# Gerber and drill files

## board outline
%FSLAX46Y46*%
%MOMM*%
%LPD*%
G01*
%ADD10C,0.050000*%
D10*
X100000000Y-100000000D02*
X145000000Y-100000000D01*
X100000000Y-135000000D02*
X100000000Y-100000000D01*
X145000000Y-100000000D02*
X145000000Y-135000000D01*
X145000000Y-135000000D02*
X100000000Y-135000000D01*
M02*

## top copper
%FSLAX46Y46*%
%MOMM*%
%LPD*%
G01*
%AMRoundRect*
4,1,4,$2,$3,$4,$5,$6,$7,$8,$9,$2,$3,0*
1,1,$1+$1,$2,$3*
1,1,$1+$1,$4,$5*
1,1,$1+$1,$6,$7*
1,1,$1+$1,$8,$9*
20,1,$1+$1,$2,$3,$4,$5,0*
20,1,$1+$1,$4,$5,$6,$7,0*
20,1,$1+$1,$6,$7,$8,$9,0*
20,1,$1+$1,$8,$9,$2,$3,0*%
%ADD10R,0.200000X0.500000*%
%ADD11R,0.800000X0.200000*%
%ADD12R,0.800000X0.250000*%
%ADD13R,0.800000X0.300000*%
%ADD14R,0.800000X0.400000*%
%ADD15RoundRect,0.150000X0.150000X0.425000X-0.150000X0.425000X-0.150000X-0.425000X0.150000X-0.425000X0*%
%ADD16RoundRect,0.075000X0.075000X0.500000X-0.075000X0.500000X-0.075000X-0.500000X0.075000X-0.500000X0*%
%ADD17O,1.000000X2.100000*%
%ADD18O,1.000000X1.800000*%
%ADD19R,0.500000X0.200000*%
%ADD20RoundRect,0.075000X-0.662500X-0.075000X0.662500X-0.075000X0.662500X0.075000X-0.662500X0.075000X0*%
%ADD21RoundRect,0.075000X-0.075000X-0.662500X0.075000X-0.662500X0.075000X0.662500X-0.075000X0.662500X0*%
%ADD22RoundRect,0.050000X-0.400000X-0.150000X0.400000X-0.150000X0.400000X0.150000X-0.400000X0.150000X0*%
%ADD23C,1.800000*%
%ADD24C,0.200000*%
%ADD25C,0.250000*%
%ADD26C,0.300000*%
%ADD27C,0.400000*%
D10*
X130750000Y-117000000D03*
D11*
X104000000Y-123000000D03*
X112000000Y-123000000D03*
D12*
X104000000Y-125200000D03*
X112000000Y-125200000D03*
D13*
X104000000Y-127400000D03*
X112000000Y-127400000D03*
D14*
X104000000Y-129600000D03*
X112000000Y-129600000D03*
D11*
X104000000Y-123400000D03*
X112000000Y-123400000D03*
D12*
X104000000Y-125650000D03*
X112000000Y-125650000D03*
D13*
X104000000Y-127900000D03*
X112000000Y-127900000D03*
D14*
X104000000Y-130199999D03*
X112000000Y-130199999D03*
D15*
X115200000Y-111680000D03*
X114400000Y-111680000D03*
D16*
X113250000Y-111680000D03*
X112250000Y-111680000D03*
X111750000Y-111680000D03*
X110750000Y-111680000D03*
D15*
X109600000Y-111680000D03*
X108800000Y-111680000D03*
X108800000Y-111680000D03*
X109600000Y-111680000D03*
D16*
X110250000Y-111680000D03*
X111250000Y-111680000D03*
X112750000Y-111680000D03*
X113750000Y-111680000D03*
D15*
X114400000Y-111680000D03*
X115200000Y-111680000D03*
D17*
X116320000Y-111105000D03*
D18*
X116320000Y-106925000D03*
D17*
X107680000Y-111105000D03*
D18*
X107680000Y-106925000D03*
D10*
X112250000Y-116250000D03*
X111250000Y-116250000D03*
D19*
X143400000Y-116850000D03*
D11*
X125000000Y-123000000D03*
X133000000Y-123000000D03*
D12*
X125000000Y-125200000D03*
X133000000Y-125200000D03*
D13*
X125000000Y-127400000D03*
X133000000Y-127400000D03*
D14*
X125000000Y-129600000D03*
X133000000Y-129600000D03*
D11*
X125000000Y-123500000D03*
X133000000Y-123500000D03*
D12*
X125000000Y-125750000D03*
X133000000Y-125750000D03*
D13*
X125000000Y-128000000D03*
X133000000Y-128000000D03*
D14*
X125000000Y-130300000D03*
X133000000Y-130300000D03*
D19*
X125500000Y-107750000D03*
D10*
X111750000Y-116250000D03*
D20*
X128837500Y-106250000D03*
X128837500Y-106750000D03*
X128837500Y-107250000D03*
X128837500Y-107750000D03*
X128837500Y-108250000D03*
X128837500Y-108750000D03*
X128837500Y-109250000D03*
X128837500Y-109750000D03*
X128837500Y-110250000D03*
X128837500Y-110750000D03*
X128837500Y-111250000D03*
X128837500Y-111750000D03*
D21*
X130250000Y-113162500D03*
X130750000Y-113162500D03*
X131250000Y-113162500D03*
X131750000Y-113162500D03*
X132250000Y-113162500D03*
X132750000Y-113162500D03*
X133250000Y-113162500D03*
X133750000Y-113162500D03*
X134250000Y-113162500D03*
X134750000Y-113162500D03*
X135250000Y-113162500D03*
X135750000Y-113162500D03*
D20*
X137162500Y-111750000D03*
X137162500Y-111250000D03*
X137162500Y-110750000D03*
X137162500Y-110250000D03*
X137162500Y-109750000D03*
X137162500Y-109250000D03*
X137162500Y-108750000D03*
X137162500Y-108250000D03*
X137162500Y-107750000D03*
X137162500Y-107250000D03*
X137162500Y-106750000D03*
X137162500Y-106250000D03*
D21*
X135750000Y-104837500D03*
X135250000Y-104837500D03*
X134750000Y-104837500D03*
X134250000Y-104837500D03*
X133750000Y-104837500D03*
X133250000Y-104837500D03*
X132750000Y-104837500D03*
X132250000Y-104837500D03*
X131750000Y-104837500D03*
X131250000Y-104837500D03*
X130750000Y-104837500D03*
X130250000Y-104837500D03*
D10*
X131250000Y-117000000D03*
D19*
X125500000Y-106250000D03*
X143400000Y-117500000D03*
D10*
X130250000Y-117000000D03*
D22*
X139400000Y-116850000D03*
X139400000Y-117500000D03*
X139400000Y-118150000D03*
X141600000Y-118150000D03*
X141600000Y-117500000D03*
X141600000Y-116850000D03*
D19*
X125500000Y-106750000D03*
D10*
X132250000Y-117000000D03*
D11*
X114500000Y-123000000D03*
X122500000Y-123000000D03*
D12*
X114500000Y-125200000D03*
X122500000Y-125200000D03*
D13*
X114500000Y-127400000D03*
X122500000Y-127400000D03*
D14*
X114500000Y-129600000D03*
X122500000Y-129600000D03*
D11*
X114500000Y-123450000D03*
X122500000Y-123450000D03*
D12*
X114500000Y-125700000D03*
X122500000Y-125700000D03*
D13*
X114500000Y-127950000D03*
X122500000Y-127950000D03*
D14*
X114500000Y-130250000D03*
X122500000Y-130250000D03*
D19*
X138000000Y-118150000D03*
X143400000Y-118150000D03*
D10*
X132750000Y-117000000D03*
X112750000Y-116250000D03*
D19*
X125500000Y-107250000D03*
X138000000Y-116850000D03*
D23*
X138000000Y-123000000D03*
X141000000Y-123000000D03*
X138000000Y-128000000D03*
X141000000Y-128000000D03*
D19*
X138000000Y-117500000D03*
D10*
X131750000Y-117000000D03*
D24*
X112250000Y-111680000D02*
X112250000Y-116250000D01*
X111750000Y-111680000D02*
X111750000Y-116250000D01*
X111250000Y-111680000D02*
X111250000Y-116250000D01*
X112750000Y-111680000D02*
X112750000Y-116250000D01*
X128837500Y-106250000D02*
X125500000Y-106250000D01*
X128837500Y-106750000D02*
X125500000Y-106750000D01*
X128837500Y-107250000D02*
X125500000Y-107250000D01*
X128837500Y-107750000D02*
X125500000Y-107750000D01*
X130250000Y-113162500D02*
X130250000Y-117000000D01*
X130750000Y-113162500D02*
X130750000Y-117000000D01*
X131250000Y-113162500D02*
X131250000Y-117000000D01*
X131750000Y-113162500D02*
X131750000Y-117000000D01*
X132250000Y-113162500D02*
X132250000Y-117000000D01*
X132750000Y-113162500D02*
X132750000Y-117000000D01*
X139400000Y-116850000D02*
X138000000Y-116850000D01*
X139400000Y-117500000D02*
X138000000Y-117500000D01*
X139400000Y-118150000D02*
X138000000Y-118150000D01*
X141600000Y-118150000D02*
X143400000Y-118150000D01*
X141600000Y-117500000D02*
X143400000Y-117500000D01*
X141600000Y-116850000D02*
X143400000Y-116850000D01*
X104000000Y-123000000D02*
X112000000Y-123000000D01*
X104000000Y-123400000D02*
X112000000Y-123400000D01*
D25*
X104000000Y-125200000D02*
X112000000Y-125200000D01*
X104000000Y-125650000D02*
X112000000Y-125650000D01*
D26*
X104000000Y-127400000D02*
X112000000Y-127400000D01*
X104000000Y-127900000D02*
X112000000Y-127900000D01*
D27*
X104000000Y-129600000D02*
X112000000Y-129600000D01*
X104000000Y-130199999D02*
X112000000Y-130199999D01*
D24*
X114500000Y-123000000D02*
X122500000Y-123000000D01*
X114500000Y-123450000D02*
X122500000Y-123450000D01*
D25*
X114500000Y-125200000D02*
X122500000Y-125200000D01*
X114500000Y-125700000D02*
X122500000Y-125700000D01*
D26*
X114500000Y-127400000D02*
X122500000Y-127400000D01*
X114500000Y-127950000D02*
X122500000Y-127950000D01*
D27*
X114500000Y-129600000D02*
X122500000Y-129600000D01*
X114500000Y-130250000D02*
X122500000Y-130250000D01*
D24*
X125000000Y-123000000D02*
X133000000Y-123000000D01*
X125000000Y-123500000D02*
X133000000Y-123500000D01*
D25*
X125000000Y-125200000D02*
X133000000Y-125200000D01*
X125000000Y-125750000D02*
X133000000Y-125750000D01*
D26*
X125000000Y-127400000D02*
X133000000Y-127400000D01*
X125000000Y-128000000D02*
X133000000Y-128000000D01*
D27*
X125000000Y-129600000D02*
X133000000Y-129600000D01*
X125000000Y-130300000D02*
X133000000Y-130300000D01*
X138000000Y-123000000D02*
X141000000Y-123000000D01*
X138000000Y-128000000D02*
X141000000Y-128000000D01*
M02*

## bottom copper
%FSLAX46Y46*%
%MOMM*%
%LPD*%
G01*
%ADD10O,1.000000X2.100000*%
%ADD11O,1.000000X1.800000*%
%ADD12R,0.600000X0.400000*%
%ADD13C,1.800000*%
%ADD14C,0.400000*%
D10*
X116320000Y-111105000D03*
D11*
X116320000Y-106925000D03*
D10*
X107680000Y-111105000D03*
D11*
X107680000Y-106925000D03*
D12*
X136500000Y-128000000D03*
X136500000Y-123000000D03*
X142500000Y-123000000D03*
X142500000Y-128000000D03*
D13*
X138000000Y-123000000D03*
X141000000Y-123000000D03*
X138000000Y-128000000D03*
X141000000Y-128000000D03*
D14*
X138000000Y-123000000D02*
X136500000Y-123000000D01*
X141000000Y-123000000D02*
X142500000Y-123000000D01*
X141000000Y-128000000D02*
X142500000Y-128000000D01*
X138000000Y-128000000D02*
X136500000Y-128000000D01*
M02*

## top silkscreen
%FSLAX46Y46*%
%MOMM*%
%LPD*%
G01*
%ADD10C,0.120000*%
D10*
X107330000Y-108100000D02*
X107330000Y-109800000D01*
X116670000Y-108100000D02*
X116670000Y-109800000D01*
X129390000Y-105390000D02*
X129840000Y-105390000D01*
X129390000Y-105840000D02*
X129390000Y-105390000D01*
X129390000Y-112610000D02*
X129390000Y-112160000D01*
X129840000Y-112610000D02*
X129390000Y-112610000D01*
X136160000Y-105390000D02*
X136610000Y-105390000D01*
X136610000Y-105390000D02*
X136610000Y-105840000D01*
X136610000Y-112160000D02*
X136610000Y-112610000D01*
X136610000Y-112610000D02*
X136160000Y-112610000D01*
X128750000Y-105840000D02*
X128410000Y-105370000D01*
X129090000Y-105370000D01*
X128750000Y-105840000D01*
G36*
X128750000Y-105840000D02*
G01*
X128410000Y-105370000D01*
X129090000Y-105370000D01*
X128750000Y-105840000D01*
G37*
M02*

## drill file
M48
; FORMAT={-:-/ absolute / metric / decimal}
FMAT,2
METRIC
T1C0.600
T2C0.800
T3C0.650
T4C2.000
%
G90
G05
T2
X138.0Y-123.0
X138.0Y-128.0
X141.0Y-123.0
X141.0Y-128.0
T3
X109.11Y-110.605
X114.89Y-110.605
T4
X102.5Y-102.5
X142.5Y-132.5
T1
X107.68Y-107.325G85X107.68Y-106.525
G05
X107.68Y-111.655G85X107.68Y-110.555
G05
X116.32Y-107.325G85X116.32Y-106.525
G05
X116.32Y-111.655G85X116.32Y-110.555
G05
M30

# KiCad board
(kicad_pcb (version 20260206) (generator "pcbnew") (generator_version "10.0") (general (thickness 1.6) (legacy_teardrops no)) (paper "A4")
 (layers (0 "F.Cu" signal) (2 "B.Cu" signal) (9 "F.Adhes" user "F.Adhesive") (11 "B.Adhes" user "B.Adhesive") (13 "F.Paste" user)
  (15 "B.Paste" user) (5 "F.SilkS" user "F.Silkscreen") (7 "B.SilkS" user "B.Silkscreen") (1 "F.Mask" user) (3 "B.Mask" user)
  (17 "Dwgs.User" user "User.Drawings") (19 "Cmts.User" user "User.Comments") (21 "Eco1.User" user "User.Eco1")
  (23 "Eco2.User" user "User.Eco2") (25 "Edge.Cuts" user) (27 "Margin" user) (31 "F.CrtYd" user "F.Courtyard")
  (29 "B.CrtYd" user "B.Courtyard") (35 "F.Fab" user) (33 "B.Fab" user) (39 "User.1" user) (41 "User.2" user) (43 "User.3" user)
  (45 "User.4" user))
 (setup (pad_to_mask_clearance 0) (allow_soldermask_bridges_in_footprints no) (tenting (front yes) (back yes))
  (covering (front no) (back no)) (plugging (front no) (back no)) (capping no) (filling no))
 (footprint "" (layer "F.Cu") (at 0 0)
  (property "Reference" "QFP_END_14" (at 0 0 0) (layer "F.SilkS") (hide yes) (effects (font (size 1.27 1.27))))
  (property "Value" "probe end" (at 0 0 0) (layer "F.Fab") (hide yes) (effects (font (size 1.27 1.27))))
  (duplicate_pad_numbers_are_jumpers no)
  (pad "1" smd rect (at 130.75 117) (size 0.2 0.5) (layers "F.Cu" "F.Mask") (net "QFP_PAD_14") (thermal_bridge_angle 45)))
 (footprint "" (layer "F.Cu") (at 0 0)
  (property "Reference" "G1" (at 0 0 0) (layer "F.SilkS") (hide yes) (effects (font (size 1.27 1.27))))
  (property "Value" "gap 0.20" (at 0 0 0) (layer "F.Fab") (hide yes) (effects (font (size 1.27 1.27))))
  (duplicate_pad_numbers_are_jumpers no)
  (pad "A0L" smd rect (at 104 123) (size 0.8 0.2) (layers "F.Cu" "F.Mask" "F.Paste") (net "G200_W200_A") (thermal_bridge_angle 45))
  (pad "A0R" smd rect (at 112 123) (size 0.8 0.2) (layers "F.Cu" "F.Mask" "F.Paste") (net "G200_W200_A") (thermal_bridge_angle 45))
  (pad "A1L" smd rect (at 104 125.2) (size 0.8 0.25) (layers "F.Cu" "F.Mask" "F.Paste") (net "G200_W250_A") (thermal_bridge_angle 45))
  (pad "A1R" smd rect (at 112 125.2) (size 0.8 0.25) (layers "F.Cu" "F.Mask" "F.Paste") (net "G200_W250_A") (thermal_bridge_angle 45))
  (pad "A2L" smd rect (at 104 127.4) (size 0.8 0.3) (layers "F.Cu" "F.Mask" "F.Paste") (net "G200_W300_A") (thermal_bridge_angle 45))
  (pad "A2R" smd rect (at 112 127.4) (size 0.8 0.3) (layers "F.Cu" "F.Mask" "F.Paste") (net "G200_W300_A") (thermal_bridge_angle 45))
  (pad "A3L" smd rect (at 104 129.6) (size 0.8 0.4) (layers "F.Cu" "F.Mask" "F.Paste") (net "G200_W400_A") (thermal_bridge_angle 45))
  (pad "A3R" smd rect (at 112 129.6) (size 0.8 0.4) (layers "F.Cu" "F.Mask" "F.Paste") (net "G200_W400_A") (thermal_bridge_angle 45))
  (pad "B0L" smd rect (at 104 123.4) (size 0.8 0.2) (layers "F.Cu" "F.Mask" "F.Paste") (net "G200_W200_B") (thermal_bridge_angle 45))
  (pad "B0R" smd rect (at 112 123.4) (size 0.8 0.2) (layers "F.Cu" "F.Mask" "F.Paste") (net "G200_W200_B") (thermal_bridge_angle 45))
  (pad "B1L" smd rect (at 104 125.65) (size 0.8 0.25) (layers "F.Cu" "F.Mask" "F.Paste") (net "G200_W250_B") (thermal_bridge_angle 45))
  (pad "B1R" smd rect (at 112 125.65) (size 0.8 0.25) (layers "F.Cu" "F.Mask" "F.Paste") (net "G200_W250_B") (thermal_bridge_angle 45))
  (pad "B2L" smd rect (at 104 127.9) (size 0.8 0.3) (layers "F.Cu" "F.Mask" "F.Paste") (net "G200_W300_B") (thermal_bridge_angle 45))
  (pad "B2R" smd rect (at 112 127.9) (size 0.8 0.3) (layers "F.Cu" "F.Mask" "F.Paste") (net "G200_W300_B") (thermal_bridge_angle 45))
  (pad "B3L" smd rect (at 104 130.199999) (size 0.8 0.4) (layers "F.Cu" "F.Mask" "F.Paste") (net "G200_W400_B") (thermal_bridge_angle 45))
  (pad "B3R" smd rect (at 112 130.199999) (size 0.8 0.4) (layers "F.Cu" "F.Mask" "F.Paste") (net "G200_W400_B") (thermal_bridge_angle 45)))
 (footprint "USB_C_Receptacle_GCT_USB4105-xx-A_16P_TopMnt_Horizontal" (layer "F.Cu") (at 112 108 180)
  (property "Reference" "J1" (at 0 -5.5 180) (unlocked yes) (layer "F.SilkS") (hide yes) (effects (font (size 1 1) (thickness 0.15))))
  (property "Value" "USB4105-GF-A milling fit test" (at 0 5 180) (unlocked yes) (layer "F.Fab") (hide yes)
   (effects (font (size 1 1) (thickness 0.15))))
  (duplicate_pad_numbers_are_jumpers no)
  (fp_line (start 4.67 -0.1) (end 4.67 -1.8) (stroke (width 0.12) (type solid)) (layer "F.SilkS"))
  (fp_line (start -4.67 -0.1) (end -4.67 -1.8) (stroke (width 0.12) (type solid)) (layer "F.SilkS"))
  (pad "" np_thru_hole circle (at -2.89 -2.605 180) (size 0.65 0.65) (drill 0.65) (layers "*.Cu" "*.Mask"))
  (pad "" np_thru_hole circle (at 2.89 -2.605 180) (size 0.65 0.65) (drill 0.65) (layers "*.Cu" "*.Mask"))
  (pad "A1" smd roundrect (at -3.2 -3.68 180) (size 0.6 1.15) (layers "F.Cu" "F.Mask" "F.Paste") (roundrect_rratio 0.25)
   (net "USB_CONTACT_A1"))
  (pad "A4" smd roundrect (at -2.4 -3.68 180) (size 0.6 1.15) (layers "F.Cu" "F.Mask" "F.Paste") (roundrect_rratio 0.25)
   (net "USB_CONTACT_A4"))
  (pad "A5" smd roundrect (at -1.25 -3.68 180) (size 0.3 1.15) (layers "F.Cu" "F.Mask" "F.Paste") (roundrect_rratio 0.25)
   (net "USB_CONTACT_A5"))
  (pad "A6" smd roundrect (at -0.25 -3.68 180) (size 0.3 1.15) (layers "F.Cu" "F.Mask" "F.Paste") (roundrect_rratio 0.25)
   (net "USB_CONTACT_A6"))
  (pad "A7" smd roundrect (at 0.25 -3.68 180) (size 0.3 1.15) (layers "F.Cu" "F.Mask" "F.Paste") (roundrect_rratio 0.25)
   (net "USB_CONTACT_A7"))
  (pad "A8" smd roundrect (at 1.25 -3.68 180) (size 0.3 1.15) (layers "F.Cu" "F.Mask" "F.Paste") (roundrect_rratio 0.25)
   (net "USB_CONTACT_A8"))
  (pad "A9" smd roundrect (at 2.4 -3.68 180) (size 0.6 1.15) (layers "F.Cu" "F.Mask" "F.Paste") (roundrect_rratio 0.25)
   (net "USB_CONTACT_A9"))
  (pad "A12" smd roundrect (at 3.2 -3.68 180) (size 0.6 1.15) (layers "F.Cu" "F.Mask" "F.Paste") (roundrect_rratio 0.25)
   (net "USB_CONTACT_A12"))
  (pad "B1" smd roundrect (at 3.2 -3.68 180) (size 0.6 1.15) (layers "F.Cu" "F.Mask" "F.Paste") (roundrect_rratio 0.25)
   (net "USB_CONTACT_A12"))
  (pad "B4" smd roundrect (at 2.4 -3.68 180) (size 0.6 1.15) (layers "F.Cu" "F.Mask" "F.Paste") (roundrect_rratio 0.25)
   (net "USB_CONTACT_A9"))
  (pad "B5" smd roundrect (at 1.75 -3.68 180) (size 0.3 1.15) (layers "F.Cu" "F.Mask" "F.Paste") (roundrect_rratio 0.25)
   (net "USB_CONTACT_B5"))
  (pad "B6" smd roundrect (at 0.75 -3.68 180) (size 0.3 1.15) (layers "F.Cu" "F.Mask" "F.Paste") (roundrect_rratio 0.25)
   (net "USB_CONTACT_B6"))
  (pad "B7" smd roundrect (at -0.75 -3.68 180) (size 0.3 1.15) (layers "F.Cu" "F.Mask" "F.Paste") (roundrect_rratio 0.25)
   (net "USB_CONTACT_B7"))
  (pad "B8" smd roundrect (at -1.75 -3.68 180) (size 0.3 1.15) (layers "F.Cu" "F.Mask" "F.Paste") (roundrect_rratio 0.25)
   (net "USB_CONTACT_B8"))
  (pad "B9" smd roundrect (at -2.4 -3.68 180) (size 0.6 1.15) (layers "F.Cu" "F.Mask" "F.Paste") (roundrect_rratio 0.25)
   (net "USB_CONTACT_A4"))
  (pad "B12" smd roundrect (at -3.2 -3.68 180) (size 0.6 1.15) (layers "F.Cu" "F.Mask" "F.Paste") (roundrect_rratio 0.25)
   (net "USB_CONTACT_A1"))
  (pad "SH" thru_hole oval (at -4.32 -3.105 180) (size 1 2.1) (drill oval 0.6 1.7) (layers "*.Cu" "*.Mask" "F.Paste")
   (remove_unused_layers no))
  (pad "SH" thru_hole oval (at -4.32 1.075 180) (size 1 1.8) (drill oval 0.6 1.4) (layers "*.Cu" "*.Mask" "F.Paste")
   (remove_unused_layers no))
  (pad "SH" thru_hole oval (at 4.32 -3.105 180) (size 1 2.1) (drill oval 0.6 1.7) (layers "*.Cu" "*.Mask" "F.Paste")
   (remove_unused_layers no))
  (pad "SH" thru_hole oval (at 4.32 1.075 180) (size 1 1.8) (drill oval 0.6 1.4) (layers "*.Cu" "*.Mask" "F.Paste")
   (remove_unused_layers no)))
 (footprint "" (layer "F.Cu") (at 0 0)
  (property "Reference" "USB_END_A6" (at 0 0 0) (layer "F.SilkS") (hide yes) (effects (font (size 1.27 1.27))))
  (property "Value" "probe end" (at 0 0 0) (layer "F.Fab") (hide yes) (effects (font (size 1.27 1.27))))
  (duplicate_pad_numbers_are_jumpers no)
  (pad "1" smd rect (at 112.25 116.25) (size 0.2 0.5) (layers "F.Cu" "F.Mask") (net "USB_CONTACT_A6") (thermal_bridge_angle 45)))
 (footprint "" (layer "F.Cu") (at 0 0)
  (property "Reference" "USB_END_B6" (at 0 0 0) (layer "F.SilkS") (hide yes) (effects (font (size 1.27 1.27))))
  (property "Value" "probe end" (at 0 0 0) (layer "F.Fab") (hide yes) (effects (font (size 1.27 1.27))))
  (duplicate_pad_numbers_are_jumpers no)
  (pad "1" smd rect (at 111.25 116.25) (size 0.2 0.5) (layers "F.Cu" "F.Mask") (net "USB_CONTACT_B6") (thermal_bridge_angle 45)))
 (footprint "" (layer "F.Cu") (at 0 0)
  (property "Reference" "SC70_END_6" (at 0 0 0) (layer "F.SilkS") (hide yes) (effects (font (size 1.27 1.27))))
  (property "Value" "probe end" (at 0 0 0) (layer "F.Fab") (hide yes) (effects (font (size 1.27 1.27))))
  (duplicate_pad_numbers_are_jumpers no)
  (pad "1" smd rect (at 143.4 116.85) (size 0.5 0.2) (layers "F.Cu" "F.Mask") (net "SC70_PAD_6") (thermal_bridge_angle 45)))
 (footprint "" (layer "F.Cu") (at 0 0)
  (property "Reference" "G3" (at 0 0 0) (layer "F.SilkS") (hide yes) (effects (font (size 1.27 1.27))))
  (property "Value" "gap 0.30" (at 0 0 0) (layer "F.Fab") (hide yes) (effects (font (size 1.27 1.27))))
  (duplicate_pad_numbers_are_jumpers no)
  (pad "A0L" smd rect (at 125 123) (size 0.8 0.2) (layers "F.Cu" "F.Mask" "F.Paste") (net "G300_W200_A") (thermal_bridge_angle 45))
  (pad "A0R" smd rect (at 133 123) (size 0.8 0.2) (layers "F.Cu" "F.Mask" "F.Paste") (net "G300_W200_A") (thermal_bridge_angle 45))
  (pad "A1L" smd rect (at 125 125.2) (size 0.8 0.25) (layers "F.Cu" "F.Mask" "F.Paste") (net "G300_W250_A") (thermal_bridge_angle 45))
  (pad "A1R" smd rect (at 133 125.2) (size 0.8 0.25) (layers "F.Cu" "F.Mask" "F.Paste") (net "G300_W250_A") (thermal_bridge_angle 45))
  (pad "A2L" smd rect (at 125 127.4) (size 0.8 0.3) (layers "F.Cu" "F.Mask" "F.Paste") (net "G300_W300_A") (thermal_bridge_angle 45))
  (pad "A2R" smd rect (at 133 127.4) (size 0.8 0.3) (layers "F.Cu" "F.Mask" "F.Paste") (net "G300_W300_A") (thermal_bridge_angle 45))
  (pad "A3L" smd rect (at 125 129.6) (size 0.8 0.4) (layers "F.Cu" "F.Mask" "F.Paste") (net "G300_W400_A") (thermal_bridge_angle 45))
  (pad "A3R" smd rect (at 133 129.6) (size 0.8 0.4) (layers "F.Cu" "F.Mask" "F.Paste") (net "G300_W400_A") (thermal_bridge_angle 45))
  (pad "B0L" smd rect (at 125 123.5) (size 0.8 0.2) (layers "F.Cu" "F.Mask" "F.Paste") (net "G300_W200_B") (thermal_bridge_angle 45))
  (pad "B0R" smd rect (at 133 123.5) (size 0.8 0.2) (layers "F.Cu" "F.Mask" "F.Paste") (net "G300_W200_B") (thermal_bridge_angle 45))
  (pad "B1L" smd rect (at 125 125.75) (size 0.8 0.25) (layers "F.Cu" "F.Mask" "F.Paste") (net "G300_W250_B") (thermal_bridge_angle 45))
  (pad "B1R" smd rect (at 133 125.75) (size 0.8 0.25) (layers "F.Cu" "F.Mask" "F.Paste") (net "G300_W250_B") (thermal_bridge_angle 45))
  (pad "B2L" smd rect (at 125 128) (size 0.8 0.3) (layers "F.Cu" "F.Mask" "F.Paste") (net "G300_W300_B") (thermal_bridge_angle 45))
  (pad "B2R" smd rect (at 133 128) (size 0.8 0.3) (layers "F.Cu" "F.Mask" "F.Paste") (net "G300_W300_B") (thermal_bridge_angle 45))
  (pad "B3L" smd rect (at 125 130.3) (size 0.8 0.4) (layers "F.Cu" "F.Mask" "F.Paste") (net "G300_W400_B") (thermal_bridge_angle 45))
  (pad "B3R" smd rect (at 133 130.3) (size 0.8 0.4) (layers "F.Cu" "F.Mask" "F.Paste") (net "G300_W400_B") (thermal_bridge_angle 45)))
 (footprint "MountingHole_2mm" (layer "F.Cu") (at 102.5 102.5)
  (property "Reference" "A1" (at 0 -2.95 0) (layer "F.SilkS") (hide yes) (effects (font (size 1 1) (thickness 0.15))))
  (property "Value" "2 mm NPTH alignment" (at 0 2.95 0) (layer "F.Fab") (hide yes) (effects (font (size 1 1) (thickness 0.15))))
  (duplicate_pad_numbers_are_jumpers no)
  (pad "" np_thru_hole circle (at 0 0) (size 2 2) (drill 2) (layers "*.Cu" "*.Mask")))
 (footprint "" (layer "F.Cu") (at 0 0)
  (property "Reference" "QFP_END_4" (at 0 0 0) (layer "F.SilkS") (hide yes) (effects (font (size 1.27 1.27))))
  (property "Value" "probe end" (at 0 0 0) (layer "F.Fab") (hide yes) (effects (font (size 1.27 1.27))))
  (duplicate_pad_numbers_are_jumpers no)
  (pad "1" smd rect (at 125.5 107.75) (size 0.5 0.2) (layers "F.Cu" "F.Mask") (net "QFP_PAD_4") (thermal_bridge_angle 45)))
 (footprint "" (layer "F.Cu") (at 0 0)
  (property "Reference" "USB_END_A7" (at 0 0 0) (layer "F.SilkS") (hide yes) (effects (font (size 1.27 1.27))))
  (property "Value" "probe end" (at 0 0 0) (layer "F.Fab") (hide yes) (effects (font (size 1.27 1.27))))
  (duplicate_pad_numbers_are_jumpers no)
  (pad "1" smd rect (at 111.75 116.25) (size 0.2 0.5) (layers "F.Cu" "F.Mask") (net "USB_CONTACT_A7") (thermal_bridge_angle 45)))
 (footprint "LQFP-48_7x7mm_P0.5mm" (layer "F.Cu") (at 133 109)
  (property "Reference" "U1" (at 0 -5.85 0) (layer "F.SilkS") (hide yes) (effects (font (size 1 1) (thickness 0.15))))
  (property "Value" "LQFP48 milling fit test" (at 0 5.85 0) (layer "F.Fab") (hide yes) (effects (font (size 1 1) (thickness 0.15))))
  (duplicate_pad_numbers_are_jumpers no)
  (fp_line (start -3.61 -3.61) (end -3.16 -3.61) (stroke (width 0.12) (type solid)) (layer "F.SilkS"))
  (fp_line (start -3.61 -3.16) (end -3.61 -3.61) (stroke (width 0.12) (type solid)) (layer "F.SilkS"))
  (fp_line (start -3.61 3.61) (end -3.61 3.16) (stroke (width 0.12) (type solid)) (layer "F.SilkS"))
  (fp_line (start -3.16 3.61) (end -3.61 3.61) (stroke (width 0.12) (type solid)) (layer "F.SilkS"))
  (fp_line (start 3.16 -3.61) (end 3.61 -3.61) (stroke (width 0.12) (type solid)) (layer "F.SilkS"))
  (fp_line (start 3.61 -3.61) (end 3.61 -3.16) (stroke (width 0.12) (type solid)) (layer "F.SilkS"))
  (fp_line (start 3.61 3.16) (end 3.61 3.61) (stroke (width 0.12) (type solid)) (layer "F.SilkS"))
  (fp_line (start 3.61 3.61) (end 3.16 3.61) (stroke (width 0.12) (type solid)) (layer "F.SilkS"))
  (fp_poly (pts (xy -4.25 -3.16) (xy -4.59 -3.63) (xy -3.91 -3.63)) (stroke (width 0.12) (type solid)) (fill yes) (layer "F.SilkS"))
  (pad "1" smd roundrect (at -4.1625 -2.75) (size 1.475 0.3) (layers "F.Cu" "F.Mask" "F.Paste") (roundrect_rratio 0.25) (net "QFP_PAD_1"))
  (pad "2" smd roundrect (at -4.1625 -2.25) (size 1.475 0.3) (layers "F.Cu" "F.Mask" "F.Paste") (roundrect_rratio 0.25) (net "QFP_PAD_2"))
  (pad "3" smd roundrect (at -4.1625 -1.75) (size 1.475 0.3) (layers "F.Cu" "F.Mask" "F.Paste") (roundrect_rratio 0.25) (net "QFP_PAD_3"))
  (pad "4" smd roundrect (at -4.1625 -1.25) (size 1.475 0.3) (layers "F.Cu" "F.Mask" "F.Paste") (roundrect_rratio 0.25) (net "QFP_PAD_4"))
  (pad "5" smd roundrect (at -4.1625 -0.75) (size 1.475 0.3) (layers "F.Cu" "F.Mask" "F.Paste") (roundrect_rratio 0.25) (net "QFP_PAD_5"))
  (pad "6" smd roundrect (at -4.1625 -0.25) (size 1.475 0.3) (layers "F.Cu" "F.Mask" "F.Paste") (roundrect_rratio 0.25) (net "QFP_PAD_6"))
  (pad "7" smd roundrect (at -4.1625 0.25) (size 1.475 0.3) (layers "F.Cu" "F.Mask" "F.Paste") (roundrect_rratio 0.25) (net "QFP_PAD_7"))
  (pad "8" smd roundrect (at -4.1625 0.75) (size 1.475 0.3) (layers "F.Cu" "F.Mask" "F.Paste") (roundrect_rratio 0.25) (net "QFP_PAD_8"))
  (pad "9" smd roundrect (at -4.1625 1.25) (size 1.475 0.3) (layers "F.Cu" "F.Mask" "F.Paste") (roundrect_rratio 0.25) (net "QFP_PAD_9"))
  (pad "10" smd roundrect (at -4.1625 1.75) (size 1.475 0.3) (layers "F.Cu" "F.Mask" "F.Paste") (roundrect_rratio 0.25) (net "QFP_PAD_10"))
  (pad "11" smd roundrect (at -4.1625 2.25) (size 1.475 0.3) (layers "F.Cu" "F.Mask" "F.Paste") (roundrect_rratio 0.25) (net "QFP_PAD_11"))
  (pad "12" smd roundrect (at -4.1625 2.75) (size 1.475 0.3) (layers "F.Cu" "F.Mask" "F.Paste") (roundrect_rratio 0.25) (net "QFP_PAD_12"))
  (pad "13" smd roundrect (at -2.75 4.1625) (size 0.3 1.475) (layers "F.Cu" "F.Mask" "F.Paste") (roundrect_rratio 0.25) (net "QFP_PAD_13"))
  (pad "14" smd roundrect (at -2.25 4.1625) (size 0.3 1.475) (layers "F.Cu" "F.Mask" "F.Paste") (roundrect_rratio 0.25) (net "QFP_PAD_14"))
  (pad "15" smd roundrect (at -1.75 4.1625) (size 0.3 1.475) (layers "F.Cu" "F.Mask" "F.Paste") (roundrect_rratio 0.25) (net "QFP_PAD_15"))
  (pad "16" smd roundrect (at -1.25 4.1625) (size 0.3 1.475) (layers "F.Cu" "F.Mask" "F.Paste") (roundrect_rratio 0.25) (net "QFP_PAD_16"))
  (pad "17" smd roundrect (at -0.75 4.1625) (size 0.3 1.475) (layers "F.Cu" "F.Mask" "F.Paste") (roundrect_rratio 0.25) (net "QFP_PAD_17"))
  (pad "18" smd roundrect (at -0.25 4.1625) (size 0.3 1.475) (layers "F.Cu" "F.Mask" "F.Paste") (roundrect_rratio 0.25) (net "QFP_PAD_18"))
  (pad "19" smd roundrect (at 0.25 4.1625) (size 0.3 1.475) (layers "F.Cu" "F.Mask" "F.Paste") (roundrect_rratio 0.25) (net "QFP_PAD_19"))
  (pad "20" smd roundrect (at 0.75 4.1625) (size 0.3 1.475) (layers "F.Cu" "F.Mask" "F.Paste") (roundrect_rratio 0.25) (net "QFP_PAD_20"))
  (pad "21" smd roundrect (at 1.25 4.1625) (size 0.3 1.475) (layers "F.Cu" "F.Mask" "F.Paste") (roundrect_rratio 0.25) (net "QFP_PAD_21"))
  (pad "22" smd roundrect (at 1.75 4.1625) (size 0.3 1.475) (layers "F.Cu" "F.Mask" "F.Paste") (roundrect_rratio 0.25) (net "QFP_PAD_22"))
  (pad "23" smd roundrect (at 2.25 4.1625) (size 0.3 1.475) (layers "F.Cu" "F.Mask" "F.Paste") (roundrect_rratio 0.25) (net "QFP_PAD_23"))
  (pad "24" smd roundrect (at 2.75 4.1625) (size 0.3 1.475) (layers "F.Cu" "F.Mask" "F.Paste") (roundrect_rratio 0.25) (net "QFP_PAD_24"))
  (pad "25" smd roundrect (at 4.1625 2.75) (size 1.475 0.3) (layers "F.Cu" "F.Mask" "F.Paste") (roundrect_rratio 0.25) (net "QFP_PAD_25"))
  (pad "26" smd roundrect (at 4.1625 2.25) (size 1.475 0.3) (layers "F.Cu" "F.Mask" "F.Paste") (roundrect_rratio 0.25) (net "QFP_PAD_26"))
  (pad "27" smd roundrect (at 4.1625 1.75) (size 1.475 0.3) (layers "F.Cu" "F.Mask" "F.Paste") (roundrect_rratio 0.25) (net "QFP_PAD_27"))
  (pad "28" smd roundrect (at 4.1625 1.25) (size 1.475 0.3) (layers "F.Cu" "F.Mask" "F.Paste") (roundrect_rratio 0.25) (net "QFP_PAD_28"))
  (pad "29" smd roundrect (at 4.1625 0.75) (size 1.475 0.3) (layers "F.Cu" "F.Mask" "F.Paste") (roundrect_rratio 0.25) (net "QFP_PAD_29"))
  (pad "30" smd roundrect (at 4.1625 0.25) (size 1.475 0.3) (layers "F.Cu" "F.Mask" "F.Paste") (roundrect_rratio 0.25) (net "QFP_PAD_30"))
  (pad "31" smd roundrect (at 4.1625 -0.25) (size 1.475 0.3) (layers "F.Cu" "F.Mask" "F.Paste") (roundrect_rratio 0.25) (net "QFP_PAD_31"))
  (pad "32" smd roundrect (at 4.1625 -0.75) (size 1.475 0.3) (layers "F.Cu" "F.Mask" "F.Paste") (roundrect_rratio 0.25) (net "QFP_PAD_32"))
  (pad "33" smd roundrect (at 4.1625 -1.25) (size 1.475 0.3) (layers "F.Cu" "F.Mask" "F.Paste") (roundrect_rratio 0.25) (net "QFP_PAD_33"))
  (pad "34" smd roundrect (at 4.1625 -1.75) (size 1.475 0.3) (layers "F.Cu" "F.Mask" "F.Paste") (roundrect_rratio 0.25) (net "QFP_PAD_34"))
  (pad "35" smd roundrect (at 4.1625 -2.25) (size 1.475 0.3) (layers "F.Cu" "F.Mask" "F.Paste") (roundrect_rratio 0.25) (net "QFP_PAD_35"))
  (pad "36" smd roundrect (at 4.1625 -2.75) (size 1.475 0.3) (layers "F.Cu" "F.Mask" "F.Paste") (roundrect_rratio 0.25) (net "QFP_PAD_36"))
  (pad "37" smd roundrect (at 2.75 -4.1625) (size 0.3 1.475) (layers "F.Cu" "F.Mask" "F.Paste") (roundrect_rratio 0.25) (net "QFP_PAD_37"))
  (pad "38" smd roundrect (at 2.25 -4.1625) (size 0.3 1.475) (layers "F.Cu" "F.Mask" "F.Paste") (roundrect_rratio 0.25) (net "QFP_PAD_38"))
  (pad "39" smd roundrect (at 1.75 -4.1625) (size 0.3 1.475) (layers "F.Cu" "F.Mask" "F.Paste") (roundrect_rratio 0.25) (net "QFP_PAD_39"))
  (pad "40" smd roundrect (at 1.25 -4.1625) (size 0.3 1.475) (layers "F.Cu" "F.Mask" "F.Paste") (roundrect_rratio 0.25) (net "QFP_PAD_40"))
  (pad "41" smd roundrect (at 0.75 -4.1625) (size 0.3 1.475) (layers "F.Cu" "F.Mask" "F.Paste") (roundrect_rratio 0.25) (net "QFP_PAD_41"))
  (pad "42" smd roundrect (at 0.25 -4.1625) (size 0.3 1.475) (layers "F.Cu" "F.Mask" "F.Paste") (roundrect_rratio 0.25) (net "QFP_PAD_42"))
  (pad "43" smd roundrect (at -0.25 -4.1625) (size 0.3 1.475) (layers "F.Cu" "F.Mask" "F.Paste") (roundrect_rratio 0.25) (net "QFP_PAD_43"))
  (pad "44" smd roundrect (at -0.75 -4.1625) (size 0.3 1.475) (layers "F.Cu" "F.Mask" "F.Paste") (roundrect_rratio 0.25) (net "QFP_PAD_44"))
  (pad "45" smd roundrect (at -1.25 -4.1625) (size 0.3 1.475) (layers "F.Cu" "F.Mask" "F.Paste") (roundrect_rratio 0.25) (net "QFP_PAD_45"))
  (pad "46" smd roundrect (at -1.75 -4.1625) (size 0.3 1.475) (layers "F.Cu" "F.Mask" "F.Paste") (roundrect_rratio 0.25) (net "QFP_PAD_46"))
  (pad "47" smd roundrect (at -2.25 -4.1625) (size 0.3 1.475) (layers "F.Cu" "F.Mask" "F.Paste") (roundrect_rratio 0.25) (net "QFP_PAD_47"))
  (pad "48" smd roundrect (at -2.75 -4.1625) (size 0.3 1.475) (layers "F.Cu" "F.Mask" "F.Paste") (roundrect_rratio 0.25) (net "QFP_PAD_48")))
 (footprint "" (layer "F.Cu") (at 0 0)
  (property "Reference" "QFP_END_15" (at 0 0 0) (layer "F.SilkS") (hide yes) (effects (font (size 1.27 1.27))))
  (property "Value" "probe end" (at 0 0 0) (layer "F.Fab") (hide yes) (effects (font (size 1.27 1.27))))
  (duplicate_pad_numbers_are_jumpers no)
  (pad "1" smd rect (at 131.25 117) (size 0.2 0.5) (layers "F.Cu" "F.Mask") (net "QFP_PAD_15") (thermal_bridge_angle 45)))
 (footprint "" (layer "F.Cu") (at 0 0)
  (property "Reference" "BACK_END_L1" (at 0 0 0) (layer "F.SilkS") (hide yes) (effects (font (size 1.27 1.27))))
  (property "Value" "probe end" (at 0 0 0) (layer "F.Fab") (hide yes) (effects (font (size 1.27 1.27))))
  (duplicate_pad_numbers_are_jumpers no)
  (pad "1" smd rect (at 136.5 128) (size 0.6 0.4) (layers "B.Cu" "B.Mask") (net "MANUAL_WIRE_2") (thermal_bridge_angle 45)))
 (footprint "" (layer "F.Cu") (at 0 0)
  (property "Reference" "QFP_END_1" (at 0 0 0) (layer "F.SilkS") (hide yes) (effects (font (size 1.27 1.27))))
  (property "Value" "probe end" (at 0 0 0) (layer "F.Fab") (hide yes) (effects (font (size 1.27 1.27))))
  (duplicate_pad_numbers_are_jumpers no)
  (pad "1" smd rect (at 125.5 106.25) (size 0.5 0.2) (layers "F.Cu" "F.Mask") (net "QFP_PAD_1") (thermal_bridge_angle 45)))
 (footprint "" (layer "F.Cu") (at 0 0)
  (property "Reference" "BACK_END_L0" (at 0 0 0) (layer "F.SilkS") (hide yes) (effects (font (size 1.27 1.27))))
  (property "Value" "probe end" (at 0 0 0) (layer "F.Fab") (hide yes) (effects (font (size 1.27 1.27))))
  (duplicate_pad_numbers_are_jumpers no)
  (pad "1" smd rect (at 136.5 123) (size 0.6 0.4) (layers "B.Cu" "B.Mask") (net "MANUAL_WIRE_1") (thermal_bridge_angle 45)))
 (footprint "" (layer "F.Cu") (at 0 0)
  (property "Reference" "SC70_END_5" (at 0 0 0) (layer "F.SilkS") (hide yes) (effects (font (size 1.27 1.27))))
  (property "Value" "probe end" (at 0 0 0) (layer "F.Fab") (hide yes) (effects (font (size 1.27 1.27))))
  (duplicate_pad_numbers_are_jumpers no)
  (pad "1" smd rect (at 143.4 117.5) (size 0.5 0.2) (layers "F.Cu" "F.Mask") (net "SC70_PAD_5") (thermal_bridge_angle 45)))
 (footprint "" (layer "F.Cu") (at 0 0)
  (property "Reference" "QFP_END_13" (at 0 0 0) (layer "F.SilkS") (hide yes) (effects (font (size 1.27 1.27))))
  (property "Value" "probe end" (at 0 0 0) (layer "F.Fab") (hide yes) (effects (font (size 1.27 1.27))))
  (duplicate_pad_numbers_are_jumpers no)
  (pad "1" smd rect (at 130.25 117) (size 0.2 0.5) (layers "F.Cu" "F.Mask") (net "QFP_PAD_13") (thermal_bridge_angle 45)))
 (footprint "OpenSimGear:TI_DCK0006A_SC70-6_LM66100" (layer "F.Cu") (at 140.5 117.5)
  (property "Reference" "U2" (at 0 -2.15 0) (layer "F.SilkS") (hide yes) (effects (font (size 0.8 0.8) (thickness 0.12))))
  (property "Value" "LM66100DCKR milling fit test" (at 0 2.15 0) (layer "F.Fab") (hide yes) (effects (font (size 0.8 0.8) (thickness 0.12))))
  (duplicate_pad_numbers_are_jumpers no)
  (pad "1" smd roundrect (at -1.1 -0.65) (size 0.9 0.4) (layers "F.Cu" "F.Mask" "F.Paste") (roundrect_rratio 0.125) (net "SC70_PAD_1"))
  (pad "2" smd roundrect (at -1.1 0) (size 0.9 0.4) (layers "F.Cu" "F.Mask" "F.Paste") (roundrect_rratio 0.125) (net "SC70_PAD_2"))
  (pad "3" smd roundrect (at -1.1 0.65) (size 0.9 0.4) (layers "F.Cu" "F.Mask" "F.Paste") (roundrect_rratio 0.125) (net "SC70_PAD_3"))
  (pad "4" smd roundrect (at 1.1 0.65) (size 0.9 0.4) (layers "F.Cu" "F.Mask" "F.Paste") (roundrect_rratio 0.125) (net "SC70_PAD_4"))
  (pad "5" smd roundrect (at 1.1 0) (size 0.9 0.4) (layers "F.Cu" "F.Mask" "F.Paste") (roundrect_rratio 0.125) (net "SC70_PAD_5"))
  (pad "6" smd roundrect (at 1.1 -0.65) (size 0.9 0.4) (layers "F.Cu" "F.Mask" "F.Paste") (roundrect_rratio 0.125) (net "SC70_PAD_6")))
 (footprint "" (layer "F.Cu") (at 0 0)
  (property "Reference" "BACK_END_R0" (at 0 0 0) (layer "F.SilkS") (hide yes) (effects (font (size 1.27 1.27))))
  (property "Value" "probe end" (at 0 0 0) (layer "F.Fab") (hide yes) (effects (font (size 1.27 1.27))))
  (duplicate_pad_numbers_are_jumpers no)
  (pad "1" smd rect (at 142.5 123) (size 0.6 0.4) (layers "B.Cu" "B.Mask") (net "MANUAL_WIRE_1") (thermal_bridge_angle 45)))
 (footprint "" (layer "F.Cu") (at 0 0)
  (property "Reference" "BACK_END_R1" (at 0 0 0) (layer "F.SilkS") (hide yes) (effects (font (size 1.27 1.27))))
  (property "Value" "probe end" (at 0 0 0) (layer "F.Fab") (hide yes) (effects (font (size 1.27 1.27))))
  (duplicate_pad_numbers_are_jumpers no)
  (pad "1" smd rect (at 142.5 128) (size 0.6 0.4) (layers "B.Cu" "B.Mask") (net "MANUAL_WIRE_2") (thermal_bridge_angle 45)))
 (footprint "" (layer "F.Cu") (at 0 0)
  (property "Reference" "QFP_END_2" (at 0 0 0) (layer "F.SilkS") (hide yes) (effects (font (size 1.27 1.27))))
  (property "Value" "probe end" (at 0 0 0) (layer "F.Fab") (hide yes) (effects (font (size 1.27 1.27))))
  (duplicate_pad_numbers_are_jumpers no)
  (pad "1" smd rect (at 125.5 106.75) (size 0.5 0.2) (layers "F.Cu" "F.Mask") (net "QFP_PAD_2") (thermal_bridge_angle 45)))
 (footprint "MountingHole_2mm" (layer "F.Cu") (at 142.5 132.5)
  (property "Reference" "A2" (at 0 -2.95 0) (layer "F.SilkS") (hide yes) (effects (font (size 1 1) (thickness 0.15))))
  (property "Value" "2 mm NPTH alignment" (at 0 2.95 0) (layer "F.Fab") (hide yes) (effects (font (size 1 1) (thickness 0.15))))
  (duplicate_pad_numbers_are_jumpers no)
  (pad "" np_thru_hole circle (at 0 0) (size 2 2) (drill 2) (layers "*.Cu" "*.Mask")))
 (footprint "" (layer "F.Cu") (at 0 0)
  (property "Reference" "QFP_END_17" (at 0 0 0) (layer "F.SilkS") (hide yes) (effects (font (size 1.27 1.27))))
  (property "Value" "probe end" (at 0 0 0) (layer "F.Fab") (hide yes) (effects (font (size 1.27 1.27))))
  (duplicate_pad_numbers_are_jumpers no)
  (pad "1" smd rect (at 132.25 117) (size 0.2 0.5) (layers "F.Cu" "F.Mask") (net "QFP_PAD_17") (thermal_bridge_angle 45)))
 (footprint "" (layer "F.Cu") (at 0 0)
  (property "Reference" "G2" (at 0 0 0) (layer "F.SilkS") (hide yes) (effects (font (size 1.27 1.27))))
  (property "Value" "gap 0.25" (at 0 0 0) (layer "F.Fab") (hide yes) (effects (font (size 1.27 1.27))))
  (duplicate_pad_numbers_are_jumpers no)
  (pad "A0L" smd rect (at 114.5 123) (size 0.8 0.2) (layers "F.Cu" "F.Mask" "F.Paste") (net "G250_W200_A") (thermal_bridge_angle 45))
  (pad "A0R" smd rect (at 122.5 123) (size 0.8 0.2) (layers "F.Cu" "F.Mask" "F.Paste") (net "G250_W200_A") (thermal_bridge_angle 45))
  (pad "A1L" smd rect (at 114.5 125.2) (size 0.8 0.25) (layers "F.Cu" "F.Mask" "F.Paste") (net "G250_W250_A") (thermal_bridge_angle 45))
  (pad "A1R" smd rect (at 122.5 125.2) (size 0.8 0.25) (layers "F.Cu" "F.Mask" "F.Paste") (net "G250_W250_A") (thermal_bridge_angle 45))
  (pad "A2L" smd rect (at 114.5 127.4) (size 0.8 0.3) (layers "F.Cu" "F.Mask" "F.Paste") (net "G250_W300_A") (thermal_bridge_angle 45))
  (pad "A2R" smd rect (at 122.5 127.4) (size 0.8 0.3) (layers "F.Cu" "F.Mask" "F.Paste") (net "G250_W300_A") (thermal_bridge_angle 45))
  (pad "A3L" smd rect (at 114.5 129.6) (size 0.8 0.4) (layers "F.Cu" "F.Mask" "F.Paste") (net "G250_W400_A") (thermal_bridge_angle 45))
  (pad "A3R" smd rect (at 122.5 129.6) (size 0.8 0.4) (layers "F.Cu" "F.Mask" "F.Paste") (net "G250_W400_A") (thermal_bridge_angle 45))
  (pad "B0L" smd rect (at 114.5 123.45) (size 0.8 0.2) (layers "F.Cu" "F.Mask" "F.Paste") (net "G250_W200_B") (thermal_bridge_angle 45))
  (pad "B0R" smd rect (at 122.5 123.45) (size 0.8 0.2) (layers "F.Cu" "F.Mask" "F.Paste") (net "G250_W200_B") (thermal_bridge_angle 45))
  (pad "B1L" smd rect (at 114.5 125.7) (size 0.8 0.25) (layers "F.Cu" "F.Mask" "F.Paste") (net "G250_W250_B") (thermal_bridge_angle 45))
  (pad "B1R" smd rect (at 122.5 125.7) (size 0.8 0.25) (layers "F.Cu" "F.Mask" "F.Paste") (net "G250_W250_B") (thermal_bridge_angle 45))
  (pad "B2L" smd rect (at 114.5 127.95) (size 0.8 0.3) (layers "F.Cu" "F.Mask" "F.Paste") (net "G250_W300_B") (thermal_bridge_angle 45))
  (pad "B2R" smd rect (at 122.5 127.95) (size 0.8 0.3) (layers "F.Cu" "F.Mask" "F.Paste") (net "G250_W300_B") (thermal_bridge_angle 45))
  (pad "B3L" smd rect (at 114.5 130.25) (size 0.8 0.4) (layers "F.Cu" "F.Mask" "F.Paste") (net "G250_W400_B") (thermal_bridge_angle 45))
  (pad "B3R" smd rect (at 122.5 130.25) (size 0.8 0.4) (layers "F.Cu" "F.Mask" "F.Paste") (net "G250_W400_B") (thermal_bridge_angle 45)))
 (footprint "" (layer "F.Cu") (at 0 0)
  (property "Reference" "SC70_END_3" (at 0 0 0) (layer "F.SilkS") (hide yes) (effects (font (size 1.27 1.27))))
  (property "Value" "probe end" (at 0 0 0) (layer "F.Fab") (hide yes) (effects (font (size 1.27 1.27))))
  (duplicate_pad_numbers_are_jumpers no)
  (pad "1" smd rect (at 138 118.15) (size 0.5 0.2) (layers "F.Cu" "F.Mask") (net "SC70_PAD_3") (thermal_bridge_angle 45)))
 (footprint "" (layer "F.Cu") (at 0 0)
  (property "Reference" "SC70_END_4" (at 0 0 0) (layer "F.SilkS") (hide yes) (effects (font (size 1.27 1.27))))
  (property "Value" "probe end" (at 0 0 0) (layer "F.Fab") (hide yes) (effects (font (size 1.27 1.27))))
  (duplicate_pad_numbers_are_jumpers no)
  (pad "1" smd rect (at 143.4 118.15) (size 0.5 0.2) (layers "F.Cu" "F.Mask") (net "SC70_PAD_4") (thermal_bridge_angle 45)))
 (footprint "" (layer "F.Cu") (at 0 0)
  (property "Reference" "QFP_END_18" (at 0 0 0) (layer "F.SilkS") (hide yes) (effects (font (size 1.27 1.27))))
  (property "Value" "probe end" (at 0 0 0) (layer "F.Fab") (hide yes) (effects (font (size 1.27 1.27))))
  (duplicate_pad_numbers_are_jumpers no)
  (pad "1" smd rect (at 132.75 117) (size 0.2 0.5) (layers "F.Cu" "F.Mask") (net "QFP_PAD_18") (thermal_bridge_angle 45)))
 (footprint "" (layer "F.Cu") (at 0 0)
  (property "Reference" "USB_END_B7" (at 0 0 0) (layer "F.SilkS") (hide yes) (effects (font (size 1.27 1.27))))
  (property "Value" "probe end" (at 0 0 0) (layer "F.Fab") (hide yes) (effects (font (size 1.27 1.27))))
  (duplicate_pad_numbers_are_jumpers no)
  (pad "1" smd rect (at 112.75 116.25) (size 0.2 0.5) (layers "F.Cu" "F.Mask") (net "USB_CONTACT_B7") (thermal_bridge_angle 45)))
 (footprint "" (layer "F.Cu") (at 0 0)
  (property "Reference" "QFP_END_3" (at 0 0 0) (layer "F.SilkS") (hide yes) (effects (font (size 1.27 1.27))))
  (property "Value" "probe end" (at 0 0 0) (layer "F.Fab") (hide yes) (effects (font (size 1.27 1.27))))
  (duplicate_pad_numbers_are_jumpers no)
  (pad "1" smd rect (at 125.5 107.25) (size 0.5 0.2) (layers "F.Cu" "F.Mask") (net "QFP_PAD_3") (thermal_bridge_angle 45)))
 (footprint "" (layer "F.Cu") (at 0 0)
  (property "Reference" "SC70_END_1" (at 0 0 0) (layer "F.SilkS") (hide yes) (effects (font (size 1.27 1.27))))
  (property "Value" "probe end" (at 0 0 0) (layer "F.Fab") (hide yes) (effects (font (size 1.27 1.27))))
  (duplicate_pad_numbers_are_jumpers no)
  (pad "1" smd rect (at 138 116.85) (size 0.5 0.2) (layers "F.Cu" "F.Mask") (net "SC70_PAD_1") (thermal_bridge_angle 45)))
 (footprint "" (layer "F.Cu") (at 0 0)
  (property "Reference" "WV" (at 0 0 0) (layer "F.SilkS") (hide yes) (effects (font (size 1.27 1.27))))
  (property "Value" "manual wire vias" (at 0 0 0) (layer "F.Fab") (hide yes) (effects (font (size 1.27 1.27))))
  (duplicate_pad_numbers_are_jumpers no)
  (pad "1" thru_hole circle (at 138 123) (size 1.8 1.8) (drill 0.8) (layers "*.Cu") (remove_unused_layers no) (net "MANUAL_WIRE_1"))
  (pad "2" thru_hole circle (at 141 123) (size 1.8 1.8) (drill 0.8) (layers "*.Cu") (remove_unused_layers no) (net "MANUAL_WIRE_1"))
  (pad "3" thru_hole circle (at 138 128) (size 1.8 1.8) (drill 0.8) (layers "*.Cu") (remove_unused_layers no) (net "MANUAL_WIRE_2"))
  (pad "4" thru_hole circle (at 141 128) (size 1.8 1.8) (drill 0.8) (layers "*.Cu") (remove_unused_layers no) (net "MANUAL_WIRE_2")))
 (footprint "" (layer "F.Cu") (at 0 0)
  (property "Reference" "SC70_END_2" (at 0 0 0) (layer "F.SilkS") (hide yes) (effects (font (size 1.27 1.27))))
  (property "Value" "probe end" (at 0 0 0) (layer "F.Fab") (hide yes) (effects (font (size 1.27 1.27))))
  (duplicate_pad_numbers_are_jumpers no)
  (pad "1" smd rect (at 138 117.5) (size 0.5 0.2) (layers "F.Cu" "F.Mask") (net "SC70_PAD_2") (thermal_bridge_angle 45)))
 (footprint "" (layer "F.Cu") (at 0 0)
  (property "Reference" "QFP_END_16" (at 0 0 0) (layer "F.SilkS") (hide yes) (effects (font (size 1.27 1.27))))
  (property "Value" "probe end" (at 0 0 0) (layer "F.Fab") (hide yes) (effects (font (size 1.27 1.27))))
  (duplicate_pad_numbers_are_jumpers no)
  (pad "1" smd rect (at 131.75 117) (size 0.2 0.5) (layers "F.Cu" "F.Mask") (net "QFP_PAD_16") (thermal_bridge_angle 45)))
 (gr_line (start 100 100) (end 145 100) (stroke (width 0.05) (type default)) (layer "Edge.Cuts"))
 (gr_line (start 100 135) (end 100 100) (stroke (width 0.05) (type default)) (layer "Edge.Cuts"))
 (gr_line (start 145 100) (end 145 135) (stroke (width 0.05) (type default)) (layer "Edge.Cuts"))
 (gr_line (start 145 135) (end 100 135) (stroke (width 0.05) (type default)) (layer "Edge.Cuts"))
 (segment (start 112.25 111.68) (end 112.25 116.25) (width 0.2) (layer "F.Cu") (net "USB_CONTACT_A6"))
 (segment (start 111.75 111.68) (end 111.75 116.25) (width 0.2) (layer "F.Cu") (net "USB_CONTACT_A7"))
 (segment (start 111.25 111.68) (end 111.25 116.25) (width 0.2) (layer "F.Cu") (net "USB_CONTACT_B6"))
 (segment (start 112.75 111.68) (end 112.75 116.25) (width 0.2) (layer "F.Cu") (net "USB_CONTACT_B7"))
 (segment (start 128.8375 106.25) (end 125.5 106.25) (width 0.2) (layer "F.Cu") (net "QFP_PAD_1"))
 (segment (start 128.8375 106.75) (end 125.5 106.75) (width 0.2) (layer "F.Cu") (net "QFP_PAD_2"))
 (segment (start 128.8375 107.25) (end 125.5 107.25) (width 0.2) (layer "F.Cu") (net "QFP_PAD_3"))
 (segment (start 128.8375 107.75) (end 125.5 107.75) (width 0.2) (layer "F.Cu") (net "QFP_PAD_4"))
 (segment (start 130.25 113.1625) (end 130.25 117) (width 0.2) (layer "F.Cu") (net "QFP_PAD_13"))
 (segment (start 130.75 113.1625) (end 130.75 117) (width 0.2) (layer "F.Cu") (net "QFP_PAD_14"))
 (segment (start 131.25 113.1625) (end 131.25 117) (width 0.2) (layer "F.Cu") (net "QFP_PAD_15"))
 (segment (start 131.75 113.1625) (end 131.75 117) (width 0.2) (layer "F.Cu") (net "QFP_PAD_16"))
 (segment (start 132.25 113.1625) (end 132.25 117) (width 0.2) (layer "F.Cu") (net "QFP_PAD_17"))
 (segment (start 132.75 113.1625) (end 132.75 117) (width 0.2) (layer "F.Cu") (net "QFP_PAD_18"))
 (segment (start 139.4 116.85) (end 138 116.85) (width 0.2) (layer "F.Cu") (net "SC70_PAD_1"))
 (segment (start 139.4 117.5) (end 138 117.5) (width 0.2) (layer "F.Cu") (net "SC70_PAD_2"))
 (segment (start 139.4 118.15) (end 138 118.15) (width 0.2) (layer "F.Cu") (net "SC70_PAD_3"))
 (segment (start 141.6 118.15) (end 143.4 118.15) (width 0.2) (layer "F.Cu") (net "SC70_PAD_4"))
 (segment (start 141.6 117.5) (end 143.4 117.5) (width 0.2) (layer "F.Cu") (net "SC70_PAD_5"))
 (segment (start 141.6 116.85) (end 143.4 116.85) (width 0.2) (layer "F.Cu") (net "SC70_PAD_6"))
 (segment (start 104 123) (end 112 123) (width 0.2) (layer "F.Cu") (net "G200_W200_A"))
 (segment (start 104 123.4) (end 112 123.4) (width 0.2) (layer "F.Cu") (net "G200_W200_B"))
 (segment (start 104 125.2) (end 112 125.2) (width 0.25) (layer "F.Cu") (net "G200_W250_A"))
 (segment (start 104 125.65) (end 112 125.65) (width 0.25) (layer "F.Cu") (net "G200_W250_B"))
 (segment (start 104 127.4) (end 112 127.4) (width 0.3) (layer "F.Cu") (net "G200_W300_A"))
 (segment (start 104 127.9) (end 112 127.9) (width 0.3) (layer "F.Cu") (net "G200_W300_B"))
 (segment (start 104 129.6) (end 112 129.6) (width 0.4) (layer "F.Cu") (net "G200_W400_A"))
 (segment (start 104 130.199999) (end 112 130.199999) (width 0.4) (layer "F.Cu") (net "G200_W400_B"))
 (segment (start 114.5 123) (end 122.5 123) (width 0.2) (layer "F.Cu") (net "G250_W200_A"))
 (segment (start 114.5 123.45) (end 122.5 123.45) (width 0.2) (layer "F.Cu") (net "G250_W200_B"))
 (segment (start 114.5 125.2) (end 122.5 125.2) (width 0.25) (layer "F.Cu") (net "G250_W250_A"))
 (segment (start 114.5 125.7) (end 122.5 125.7) (width 0.25) (layer "F.Cu") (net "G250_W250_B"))
 (segment (start 114.5 127.4) (end 122.5 127.4) (width 0.3) (layer "F.Cu") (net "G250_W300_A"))
 (segment (start 114.5 127.95) (end 122.5 127.95) (width 0.3) (layer "F.Cu") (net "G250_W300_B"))
 (segment (start 114.5 129.6) (end 122.5 129.6) (width 0.4) (layer "F.Cu") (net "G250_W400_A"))
 (segment (start 114.5 130.25) (end 122.5 130.25) (width 0.4) (layer "F.Cu") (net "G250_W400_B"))
 (segment (start 125 123) (end 133 123) (width 0.2) (layer "F.Cu") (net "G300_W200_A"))
 (segment (start 125 123.5) (end 133 123.5) (width 0.2) (layer "F.Cu") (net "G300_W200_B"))
 (segment (start 125 125.2) (end 133 125.2) (width 0.25) (layer "F.Cu") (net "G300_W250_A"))
 (segment (start 125 125.75) (end 133 125.75) (width 0.25) (layer "F.Cu") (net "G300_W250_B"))
 (segment (start 125 127.4) (end 133 127.4) (width 0.3) (layer "F.Cu") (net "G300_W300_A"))
 (segment (start 125 128) (end 133 128) (width 0.3) (layer "F.Cu") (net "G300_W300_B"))
 (segment (start 125 129.6) (end 133 129.6) (width 0.4) (layer "F.Cu") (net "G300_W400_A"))
 (segment (start 125 130.3) (end 133 130.3) (width 0.4) (layer "F.Cu") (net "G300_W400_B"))
 (segment (start 138 123) (end 141 123) (width 0.4) (layer "F.Cu") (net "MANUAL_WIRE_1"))
 (segment (start 138 123) (end 136.5 123) (width 0.4) (layer "B.Cu") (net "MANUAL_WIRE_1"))
 (segment (start 141 123) (end 142.5 123) (width 0.4) (layer "B.Cu") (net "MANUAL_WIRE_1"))
 (segment (start 138 128) (end 141 128) (width 0.4) (layer "F.Cu") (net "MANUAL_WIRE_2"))
 (segment (start 141 128) (end 142.5 128) (width 0.4) (layer "B.Cu") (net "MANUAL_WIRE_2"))
 (segment (start 138 128) (end 136.5 128) (width 0.4) (layer "B.Cu") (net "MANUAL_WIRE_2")))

